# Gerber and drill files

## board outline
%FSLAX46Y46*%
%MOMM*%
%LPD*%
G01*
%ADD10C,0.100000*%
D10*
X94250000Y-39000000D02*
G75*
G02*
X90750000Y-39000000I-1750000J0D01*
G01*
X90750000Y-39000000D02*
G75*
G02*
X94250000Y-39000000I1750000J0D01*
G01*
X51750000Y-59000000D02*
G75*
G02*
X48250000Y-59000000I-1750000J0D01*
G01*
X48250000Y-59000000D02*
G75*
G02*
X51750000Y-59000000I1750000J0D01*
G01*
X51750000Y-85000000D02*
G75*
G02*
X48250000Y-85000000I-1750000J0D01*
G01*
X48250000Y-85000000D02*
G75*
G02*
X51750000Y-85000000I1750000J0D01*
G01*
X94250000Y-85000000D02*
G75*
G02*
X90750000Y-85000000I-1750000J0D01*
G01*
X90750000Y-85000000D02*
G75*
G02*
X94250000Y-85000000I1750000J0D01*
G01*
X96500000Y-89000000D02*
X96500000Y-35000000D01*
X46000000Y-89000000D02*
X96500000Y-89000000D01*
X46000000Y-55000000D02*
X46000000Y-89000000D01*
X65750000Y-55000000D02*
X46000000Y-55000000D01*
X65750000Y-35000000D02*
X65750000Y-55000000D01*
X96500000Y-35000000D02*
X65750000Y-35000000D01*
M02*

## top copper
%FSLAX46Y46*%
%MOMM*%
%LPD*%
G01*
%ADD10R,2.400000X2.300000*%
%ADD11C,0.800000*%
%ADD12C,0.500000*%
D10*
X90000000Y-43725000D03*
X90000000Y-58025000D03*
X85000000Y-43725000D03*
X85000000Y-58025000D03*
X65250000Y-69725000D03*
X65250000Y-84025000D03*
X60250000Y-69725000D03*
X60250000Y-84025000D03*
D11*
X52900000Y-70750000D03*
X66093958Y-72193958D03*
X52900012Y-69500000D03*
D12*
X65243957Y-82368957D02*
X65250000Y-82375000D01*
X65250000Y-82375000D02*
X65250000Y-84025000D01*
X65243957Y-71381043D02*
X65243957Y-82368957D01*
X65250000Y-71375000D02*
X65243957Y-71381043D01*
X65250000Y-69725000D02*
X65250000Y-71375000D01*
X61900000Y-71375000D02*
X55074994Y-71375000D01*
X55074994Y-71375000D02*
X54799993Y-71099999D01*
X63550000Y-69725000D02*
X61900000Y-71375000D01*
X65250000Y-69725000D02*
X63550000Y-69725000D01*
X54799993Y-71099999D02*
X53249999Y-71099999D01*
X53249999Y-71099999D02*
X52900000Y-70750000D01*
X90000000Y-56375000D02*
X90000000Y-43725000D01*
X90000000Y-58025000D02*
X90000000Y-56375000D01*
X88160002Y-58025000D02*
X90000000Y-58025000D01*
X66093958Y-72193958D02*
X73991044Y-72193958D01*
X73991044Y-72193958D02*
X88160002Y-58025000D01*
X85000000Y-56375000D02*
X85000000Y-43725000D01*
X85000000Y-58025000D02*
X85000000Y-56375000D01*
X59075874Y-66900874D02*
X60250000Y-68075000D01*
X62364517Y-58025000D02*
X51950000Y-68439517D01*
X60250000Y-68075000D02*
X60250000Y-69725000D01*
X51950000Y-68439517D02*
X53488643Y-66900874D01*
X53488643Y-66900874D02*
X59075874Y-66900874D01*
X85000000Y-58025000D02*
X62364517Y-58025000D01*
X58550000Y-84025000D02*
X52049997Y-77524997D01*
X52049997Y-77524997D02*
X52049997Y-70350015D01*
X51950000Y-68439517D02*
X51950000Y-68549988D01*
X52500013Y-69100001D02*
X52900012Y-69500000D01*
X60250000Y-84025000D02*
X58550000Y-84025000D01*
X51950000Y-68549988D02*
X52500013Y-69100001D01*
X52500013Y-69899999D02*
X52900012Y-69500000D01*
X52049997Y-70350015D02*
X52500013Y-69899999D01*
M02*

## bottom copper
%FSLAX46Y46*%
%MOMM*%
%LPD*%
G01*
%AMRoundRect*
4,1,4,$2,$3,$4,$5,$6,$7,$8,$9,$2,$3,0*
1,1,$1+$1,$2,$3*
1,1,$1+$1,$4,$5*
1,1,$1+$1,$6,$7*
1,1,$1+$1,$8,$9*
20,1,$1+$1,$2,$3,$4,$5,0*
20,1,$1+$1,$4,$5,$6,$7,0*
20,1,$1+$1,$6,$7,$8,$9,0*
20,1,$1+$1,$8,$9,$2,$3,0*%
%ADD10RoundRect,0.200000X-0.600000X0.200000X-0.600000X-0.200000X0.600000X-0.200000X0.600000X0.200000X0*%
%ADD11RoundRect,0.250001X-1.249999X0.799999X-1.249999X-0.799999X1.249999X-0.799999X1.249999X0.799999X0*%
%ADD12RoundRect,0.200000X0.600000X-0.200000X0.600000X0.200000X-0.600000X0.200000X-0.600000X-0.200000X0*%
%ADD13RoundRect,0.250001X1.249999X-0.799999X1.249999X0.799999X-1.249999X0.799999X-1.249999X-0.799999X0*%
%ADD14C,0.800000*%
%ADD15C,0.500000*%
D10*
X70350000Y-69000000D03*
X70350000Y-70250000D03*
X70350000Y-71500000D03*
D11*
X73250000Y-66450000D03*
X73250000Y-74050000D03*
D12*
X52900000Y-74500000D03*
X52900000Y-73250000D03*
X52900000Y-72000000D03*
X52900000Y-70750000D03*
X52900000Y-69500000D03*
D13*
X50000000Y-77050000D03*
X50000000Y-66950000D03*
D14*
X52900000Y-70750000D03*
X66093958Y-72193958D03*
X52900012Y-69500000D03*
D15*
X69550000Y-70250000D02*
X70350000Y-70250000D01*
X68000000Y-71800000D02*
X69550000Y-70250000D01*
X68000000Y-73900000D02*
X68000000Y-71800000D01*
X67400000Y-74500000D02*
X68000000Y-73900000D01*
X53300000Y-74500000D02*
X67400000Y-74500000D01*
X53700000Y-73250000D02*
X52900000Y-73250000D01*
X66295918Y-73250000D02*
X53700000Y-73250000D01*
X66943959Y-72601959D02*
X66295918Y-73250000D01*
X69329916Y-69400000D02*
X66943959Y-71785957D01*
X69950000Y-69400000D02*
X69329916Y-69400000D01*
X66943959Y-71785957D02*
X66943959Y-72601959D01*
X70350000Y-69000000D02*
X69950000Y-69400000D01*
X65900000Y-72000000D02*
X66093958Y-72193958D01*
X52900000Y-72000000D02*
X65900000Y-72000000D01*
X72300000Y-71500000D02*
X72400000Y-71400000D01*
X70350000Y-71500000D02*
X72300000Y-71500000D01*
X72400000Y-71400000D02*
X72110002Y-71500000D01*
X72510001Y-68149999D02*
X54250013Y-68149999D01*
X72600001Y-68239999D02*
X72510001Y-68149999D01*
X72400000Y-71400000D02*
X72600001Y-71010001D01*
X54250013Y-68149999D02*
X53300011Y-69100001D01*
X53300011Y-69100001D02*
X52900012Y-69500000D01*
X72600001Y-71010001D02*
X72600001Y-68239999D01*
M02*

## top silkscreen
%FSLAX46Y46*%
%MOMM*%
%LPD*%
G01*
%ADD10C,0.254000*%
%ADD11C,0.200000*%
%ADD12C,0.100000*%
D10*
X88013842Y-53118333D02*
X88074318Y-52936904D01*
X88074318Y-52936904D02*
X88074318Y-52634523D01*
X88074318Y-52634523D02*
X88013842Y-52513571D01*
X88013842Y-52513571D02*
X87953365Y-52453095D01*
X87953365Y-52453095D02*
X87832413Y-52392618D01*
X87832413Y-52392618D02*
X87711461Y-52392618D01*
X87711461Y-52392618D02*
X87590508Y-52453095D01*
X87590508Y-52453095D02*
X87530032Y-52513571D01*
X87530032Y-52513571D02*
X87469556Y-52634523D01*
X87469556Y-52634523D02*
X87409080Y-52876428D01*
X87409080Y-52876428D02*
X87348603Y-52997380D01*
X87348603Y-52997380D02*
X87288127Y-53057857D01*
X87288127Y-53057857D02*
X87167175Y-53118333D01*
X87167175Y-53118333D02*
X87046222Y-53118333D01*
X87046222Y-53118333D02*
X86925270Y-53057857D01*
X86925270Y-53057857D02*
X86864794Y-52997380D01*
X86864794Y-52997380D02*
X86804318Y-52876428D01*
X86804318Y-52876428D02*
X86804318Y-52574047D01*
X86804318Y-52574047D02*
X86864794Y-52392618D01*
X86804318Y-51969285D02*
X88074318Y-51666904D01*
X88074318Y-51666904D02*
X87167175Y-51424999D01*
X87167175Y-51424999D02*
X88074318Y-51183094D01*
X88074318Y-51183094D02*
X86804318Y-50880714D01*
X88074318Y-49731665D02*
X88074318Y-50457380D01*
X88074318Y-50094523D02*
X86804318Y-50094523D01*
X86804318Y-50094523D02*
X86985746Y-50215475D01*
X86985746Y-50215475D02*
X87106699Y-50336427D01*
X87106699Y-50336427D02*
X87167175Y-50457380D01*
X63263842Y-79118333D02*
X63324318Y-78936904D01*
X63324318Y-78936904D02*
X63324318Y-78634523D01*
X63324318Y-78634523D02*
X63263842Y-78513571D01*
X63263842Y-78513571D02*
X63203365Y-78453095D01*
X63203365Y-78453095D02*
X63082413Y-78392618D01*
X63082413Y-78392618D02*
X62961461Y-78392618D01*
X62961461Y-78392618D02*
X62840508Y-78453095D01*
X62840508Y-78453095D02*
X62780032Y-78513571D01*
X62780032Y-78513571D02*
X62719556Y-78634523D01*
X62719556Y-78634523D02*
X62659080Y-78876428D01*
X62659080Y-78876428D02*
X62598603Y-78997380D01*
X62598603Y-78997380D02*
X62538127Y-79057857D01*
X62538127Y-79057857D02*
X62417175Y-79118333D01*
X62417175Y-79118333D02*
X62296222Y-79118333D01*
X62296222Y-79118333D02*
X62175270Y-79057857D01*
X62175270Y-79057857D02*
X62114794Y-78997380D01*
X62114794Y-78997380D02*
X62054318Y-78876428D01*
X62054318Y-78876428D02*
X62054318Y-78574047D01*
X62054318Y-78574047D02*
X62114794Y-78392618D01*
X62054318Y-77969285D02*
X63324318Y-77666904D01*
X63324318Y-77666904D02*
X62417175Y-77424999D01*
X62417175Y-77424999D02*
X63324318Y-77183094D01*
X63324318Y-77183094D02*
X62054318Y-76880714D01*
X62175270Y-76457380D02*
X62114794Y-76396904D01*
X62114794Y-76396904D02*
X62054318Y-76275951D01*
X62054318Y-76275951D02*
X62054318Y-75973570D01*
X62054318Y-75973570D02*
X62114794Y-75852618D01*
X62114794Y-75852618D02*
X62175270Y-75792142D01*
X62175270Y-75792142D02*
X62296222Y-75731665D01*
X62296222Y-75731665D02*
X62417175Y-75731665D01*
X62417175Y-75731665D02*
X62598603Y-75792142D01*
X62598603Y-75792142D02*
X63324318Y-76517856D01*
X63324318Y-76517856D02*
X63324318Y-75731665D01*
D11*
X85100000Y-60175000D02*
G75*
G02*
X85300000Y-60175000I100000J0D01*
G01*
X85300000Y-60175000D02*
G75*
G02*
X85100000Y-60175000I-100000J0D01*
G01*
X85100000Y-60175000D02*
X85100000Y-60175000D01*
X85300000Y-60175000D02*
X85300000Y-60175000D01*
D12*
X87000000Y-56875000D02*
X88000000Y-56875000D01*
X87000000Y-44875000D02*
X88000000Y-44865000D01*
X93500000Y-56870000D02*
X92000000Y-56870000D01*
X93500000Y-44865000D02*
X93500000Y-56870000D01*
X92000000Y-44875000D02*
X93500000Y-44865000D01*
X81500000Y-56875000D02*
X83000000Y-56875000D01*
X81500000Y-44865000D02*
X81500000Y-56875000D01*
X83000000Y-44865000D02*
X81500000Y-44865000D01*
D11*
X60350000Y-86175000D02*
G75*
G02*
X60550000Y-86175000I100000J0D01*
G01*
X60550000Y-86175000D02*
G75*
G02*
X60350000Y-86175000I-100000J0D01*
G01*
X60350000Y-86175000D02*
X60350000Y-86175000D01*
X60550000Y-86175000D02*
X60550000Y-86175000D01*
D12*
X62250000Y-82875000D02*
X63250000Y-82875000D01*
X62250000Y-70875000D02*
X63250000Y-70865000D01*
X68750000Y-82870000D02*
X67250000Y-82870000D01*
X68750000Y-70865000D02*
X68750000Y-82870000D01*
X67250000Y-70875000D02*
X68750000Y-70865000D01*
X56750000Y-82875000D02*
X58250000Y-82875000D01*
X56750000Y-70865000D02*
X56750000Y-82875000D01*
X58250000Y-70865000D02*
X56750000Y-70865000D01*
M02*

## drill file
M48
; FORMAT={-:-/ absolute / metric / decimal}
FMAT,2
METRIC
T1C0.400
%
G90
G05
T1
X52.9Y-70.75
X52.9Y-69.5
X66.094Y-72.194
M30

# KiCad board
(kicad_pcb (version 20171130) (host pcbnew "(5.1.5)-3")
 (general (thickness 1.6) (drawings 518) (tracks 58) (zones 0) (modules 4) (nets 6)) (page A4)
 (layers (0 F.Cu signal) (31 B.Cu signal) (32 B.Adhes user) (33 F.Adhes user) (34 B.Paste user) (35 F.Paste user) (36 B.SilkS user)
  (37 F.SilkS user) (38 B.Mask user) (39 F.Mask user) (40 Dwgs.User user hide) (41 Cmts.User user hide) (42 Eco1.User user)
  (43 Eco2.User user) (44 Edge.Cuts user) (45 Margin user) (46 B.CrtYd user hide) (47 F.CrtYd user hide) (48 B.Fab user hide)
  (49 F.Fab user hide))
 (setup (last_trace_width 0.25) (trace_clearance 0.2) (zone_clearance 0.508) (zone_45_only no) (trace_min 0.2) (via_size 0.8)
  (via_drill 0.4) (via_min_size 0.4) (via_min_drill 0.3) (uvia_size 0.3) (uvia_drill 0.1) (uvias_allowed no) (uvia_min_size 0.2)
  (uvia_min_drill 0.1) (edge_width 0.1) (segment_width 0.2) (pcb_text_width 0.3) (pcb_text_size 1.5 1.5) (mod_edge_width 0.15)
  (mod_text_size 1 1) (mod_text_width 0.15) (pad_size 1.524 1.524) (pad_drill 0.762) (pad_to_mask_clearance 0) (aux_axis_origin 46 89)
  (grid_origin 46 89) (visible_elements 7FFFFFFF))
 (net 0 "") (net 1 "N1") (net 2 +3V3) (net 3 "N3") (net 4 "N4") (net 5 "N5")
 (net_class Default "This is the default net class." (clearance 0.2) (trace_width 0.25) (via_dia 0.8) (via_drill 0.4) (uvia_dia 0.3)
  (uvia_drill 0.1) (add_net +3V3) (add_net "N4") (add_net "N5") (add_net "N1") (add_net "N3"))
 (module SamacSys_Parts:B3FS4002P (layer F.Cu) (at 87.5 52 270)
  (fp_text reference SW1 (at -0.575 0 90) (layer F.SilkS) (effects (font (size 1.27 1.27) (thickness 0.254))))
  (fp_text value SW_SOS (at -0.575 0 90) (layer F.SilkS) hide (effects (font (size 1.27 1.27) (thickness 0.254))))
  (fp_arc (start 8.175 2.3) (end 8.175 2.4) (angle 180) (layer F.SilkS) (width 0.2))
  (fp_arc (start 8.175 2.3) (end 8.175 2.2) (angle 180) (layer F.SilkS) (width 0.2))
  (fp_line (start 8.175 2.4) (end 8.175 2.4) (layer F.SilkS) (width 0.2))
  (fp_line (start 8.175 2.2) (end 8.175 2.2) (layer F.SilkS) (width 0.2))
  (fp_line (start 4.875 0.5) (end 4.875 -0.5) (layer F.SilkS) (width 0.1))
  (fp_line (start -7.125 0.5) (end -7.135 -0.5) (layer F.SilkS) (width 0.1))
  (fp_line (start 4.87 -6) (end 4.87 -4.5) (layer F.SilkS) (width 0.1))
  (fp_line (start -7.135 -6) (end 4.87 -6) (layer F.SilkS) (width 0.1))
  (fp_line (start -7.125 -4.5) (end -7.135 -6) (layer F.SilkS) (width 0.1))
  (fp_line (start 4.875 6) (end 4.875 4.5) (layer F.SilkS) (width 0.1))
  (fp_line (start -7.135 6) (end 4.875 6) (layer F.SilkS) (width 0.1))
  (fp_line (start -7.135 4.5) (end -7.135 6) (layer F.SilkS) (width 0.1))
  (pad 2 smd rect (at -8.275 -2.5 270) (size 2.3 2.4) (layers F.Cu F.Paste F.Mask) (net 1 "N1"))
  (pad 2 smd rect (at 6.025 -2.5 270) (size 2.3 2.4) (layers F.Cu F.Paste F.Mask) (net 1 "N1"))
  (pad 1 smd rect (at -8.275 2.5 270) (size 2.3 2.4) (layers F.Cu F.Paste F.Mask) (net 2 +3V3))
  (pad 1 smd rect (at 6.025 2.5 270) (size 2.3 2.4) (layers F.Cu F.Paste F.Mask) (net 2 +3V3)))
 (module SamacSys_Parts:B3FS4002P (layer F.Cu) (at 62.75 78 270)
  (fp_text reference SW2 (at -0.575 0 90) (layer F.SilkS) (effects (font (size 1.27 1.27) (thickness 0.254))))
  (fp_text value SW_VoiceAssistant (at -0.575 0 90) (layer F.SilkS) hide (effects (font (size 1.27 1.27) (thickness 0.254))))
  (fp_arc (start 8.175 2.3) (end 8.175 2.4) (angle 180) (layer F.SilkS) (width 0.2))
  (fp_arc (start 8.175 2.3) (end 8.175 2.2) (angle 180) (layer F.SilkS) (width 0.2))
  (fp_line (start 8.175 2.4) (end 8.175 2.4) (layer F.SilkS) (width 0.2))
  (fp_line (start 8.175 2.2) (end 8.175 2.2) (layer F.SilkS) (width 0.2))
  (fp_line (start 4.875 0.5) (end 4.875 -0.5) (layer F.SilkS) (width 0.1))
  (fp_line (start -7.125 0.5) (end -7.135 -0.5) (layer F.SilkS) (width 0.1))
  (fp_line (start 4.87 -6) (end 4.87 -4.5) (layer F.SilkS) (width 0.1))
  (fp_line (start -7.135 -6) (end 4.87 -6) (layer F.SilkS) (width 0.1))
  (fp_line (start -7.125 -4.5) (end -7.135 -6) (layer F.SilkS) (width 0.1))
  (fp_line (start 4.875 6) (end 4.875 4.5) (layer F.SilkS) (width 0.1))
  (fp_line (start -7.135 6) (end 4.875 6) (layer F.SilkS) (width 0.1))
  (fp_line (start -7.135 4.5) (end -7.135 6) (layer F.SilkS) (width 0.1))
  (pad 2 smd rect (at -8.275 -2.5 270) (size 2.3 2.4) (layers F.Cu F.Paste F.Mask) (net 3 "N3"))
  (pad 2 smd rect (at 6.025 -2.5 270) (size 2.3 2.4) (layers F.Cu F.Paste F.Mask) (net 3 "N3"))
  (pad 1 smd rect (at -8.275 2.5 270) (size 2.3 2.4) (layers F.Cu F.Paste F.Mask) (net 2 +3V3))
  (pad 1 smd rect (at 6.025 2.5 270) (size 2.3 2.4) (layers F.Cu F.Paste F.Mask) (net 2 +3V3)))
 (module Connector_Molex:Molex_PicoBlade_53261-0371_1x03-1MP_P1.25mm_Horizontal (layer B.Cu) (at 72.75 70.25 270)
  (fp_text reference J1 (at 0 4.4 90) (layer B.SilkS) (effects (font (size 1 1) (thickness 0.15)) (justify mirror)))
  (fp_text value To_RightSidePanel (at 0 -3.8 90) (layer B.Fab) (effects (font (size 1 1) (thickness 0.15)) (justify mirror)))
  (pad 1 smd roundrect (at -1.25 2.4 270) (size 0.8 1.6) (layers B.Cu B.Paste B.Mask) (roundrect_rratio 0.25) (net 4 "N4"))
  (pad 2 smd roundrect (at 0 2.4 270) (size 0.8 1.6) (layers B.Cu B.Paste B.Mask) (roundrect_rratio 0.25) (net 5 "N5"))
  (pad 3 smd roundrect (at 1.25 2.4 270) (size 0.8 1.6) (layers B.Cu B.Paste B.Mask) (roundrect_rratio 0.25) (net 2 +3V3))
  (pad MP smd roundrect (at -3.8 -0.5 270) (size 2.1 3) (layers B.Cu B.Paste B.Mask) (roundrect_rratio 0.119048))
  (pad MP smd roundrect (at 3.8 -0.5 270) (size 2.1 3) (layers B.Cu B.Paste B.Mask) (roundrect_rratio 0.119048)))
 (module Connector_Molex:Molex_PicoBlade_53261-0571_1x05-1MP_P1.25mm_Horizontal (layer B.Cu) (at 50.5 72 90)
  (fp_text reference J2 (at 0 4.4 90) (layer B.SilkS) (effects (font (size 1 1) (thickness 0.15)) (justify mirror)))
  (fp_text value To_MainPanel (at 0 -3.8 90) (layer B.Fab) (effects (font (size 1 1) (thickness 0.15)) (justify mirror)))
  (pad 1 smd roundrect (at -2.5 2.4 90) (size 0.8 1.6) (layers B.Cu B.Paste B.Mask) (roundrect_rratio 0.25) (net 5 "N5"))
  (pad 2 smd roundrect (at -1.25 2.4 90) (size 0.8 1.6) (layers B.Cu B.Paste B.Mask) (roundrect_rratio 0.25) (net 4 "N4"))
  (pad 3 smd roundrect (at 0 2.4 90) (size 0.8 1.6) (layers B.Cu B.Paste B.Mask) (roundrect_rratio 0.25) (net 1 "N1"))
  (pad 4 smd roundrect (at 1.25 2.4 90) (size 0.8 1.6) (layers B.Cu B.Paste B.Mask) (roundrect_rratio 0.25) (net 3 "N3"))
  (pad 5 smd roundrect (at 2.5 2.4 90) (size 0.8 1.6) (layers B.Cu B.Paste B.Mask) (roundrect_rratio 0.25) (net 2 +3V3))
  (pad MP smd roundrect (at -5.05 -0.5 90) (size 2.1 3) (layers B.Cu B.Paste B.Mask) (roundrect_rratio 0.119048))
  (pad MP smd roundrect (at 5.05 -0.5 90) (size 2.1 3) (layers B.Cu B.Paste B.Mask) (roundrect_rratio 0.119048)))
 (gr_circle (center 92.5 39) (end 92.5 37.25) (layer Edge.Cuts) (width 0.1))
 (gr_circle (center 50 59) (end 48.25 59) (layer Edge.Cuts) (width 0.1))
 (gr_circle (center 50 85) (end 48.25 85) (layer Edge.Cuts) (width 0.1))
 (gr_circle (center 92.5 85) (end 90.75 85) (layer Edge.Cuts) (width 0.1))
 (gr_line (start 96.5 89) (end 96.5 35) (layer Edge.Cuts) (width 0.1))
 (gr_line (start 46 89) (end 96.5 89) (layer Edge.Cuts) (width 0.1))
 (gr_line (start 46 55) (end 46 89) (layer Edge.Cuts) (width 0.1))
 (gr_line (start 65.75 55) (end 46 55) (layer Edge.Cuts) (width 0.1))
 (gr_line (start 65.75 35) (end 65.75 55) (layer Edge.Cuts) (width 0.1))
 (gr_line (start 96.5 35) (end 65.75 35) (layer Edge.Cuts) (width 0.1))
 (segment (start 69.55 70.25) (end 70.35 70.25) (width 0.5) (layer B.Cu) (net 5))
 (segment (start 68 71.8) (end 69.55 70.25) (width 0.5) (layer B.Cu) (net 5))
 (segment (start 68 73.9) (end 68 71.8) (width 0.5) (layer B.Cu) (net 5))
 (segment (start 67.4 74.5) (end 68 73.9) (width 0.5) (layer B.Cu) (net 5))
 (segment (start 53.3 74.5) (end 67.4 74.5) (width 0.5) (layer B.Cu) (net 5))
 (segment (start 53.7 73.25) (end 52.9 73.25) (width 0.5) (layer B.Cu) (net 4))
 (segment (start 66.295918 73.25) (end 53.7 73.25) (width 0.5) (layer B.Cu) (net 4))
 (segment (start 66.943959 72.601959) (end 66.295918 73.25) (width 0.5) (layer B.Cu) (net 4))
 (segment (start 69.329916 69.4) (end 66.943959 71.785957) (width 0.5) (layer B.Cu) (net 4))
 (segment (start 69.95 69.4) (end 69.329916 69.4) (width 0.5) (layer B.Cu) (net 4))
 (segment (start 66.943959 71.785957) (end 66.943959 72.601959) (width 0.5) (layer B.Cu) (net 4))
 (segment (start 70.35 69) (end 69.95 69.4) (width 0.5) (layer B.Cu) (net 4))
 (segment (start 65.243957 82.368957) (end 65.25 82.375) (width 0.5) (layer F.Cu) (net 3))
 (segment (start 65.25 82.375) (end 65.25 84.025) (width 0.5) (layer F.Cu) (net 3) (status 20))
 (segment (start 65.243957 71.381043) (end 65.243957 82.368957) (width 0.5) (layer F.Cu) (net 3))
 (segment (start 65.25 71.375) (end 65.243957 71.381043) (width 0.5) (layer F.Cu) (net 3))
 (segment (start 65.25 69.725) (end 65.25 71.375) (width 0.5) (layer F.Cu) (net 3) (status 10))
 (segment (start 61.9 71.375) (end 55.074994 71.375) (width 0.5) (layer F.Cu) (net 3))
 (segment (start 55.074994 71.375) (end 54.799993 71.099999) (width 0.5) (layer F.Cu) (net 3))
 (segment (start 63.55 69.725) (end 61.9 71.375) (width 0.5) (layer F.Cu) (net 3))
 (segment (start 65.25 69.725) (end 63.55 69.725) (width 0.5) (layer F.Cu) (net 3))
 (via (at 52.9 70.75) (size 0.8) (drill 0.4) (layers F.Cu B.Cu) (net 3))
 (segment (start 54.799993 71.099999) (end 53.249999 71.099999) (width 0.5) (layer F.Cu) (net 3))
 (segment (start 53.249999 71.099999) (end 52.9 70.75) (width 0.5) (layer F.Cu) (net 3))
 (segment (start 90 56.375) (end 90 43.725) (width 0.5) (layer F.Cu) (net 1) (status 20))
 (segment (start 90 58.025) (end 90 56.375) (width 0.5) (layer F.Cu) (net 1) (status 10))
 (via (at 66.093958 72.193958) (size 0.8) (drill 0.4) (layers F.Cu B.Cu) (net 1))
 (segment (start 88.160002 58.025) (end 90 58.025) (width 0.5) (layer F.Cu) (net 1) (status 20))
 (segment (start 66.093958 72.193958) (end 73.991044 72.193958) (width 0.5) (layer F.Cu) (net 1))
 (segment (start 73.991044 72.193958) (end 88.160002 58.025) (width 0.5) (layer F.Cu) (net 1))
 (segment (start 65.9 72) (end 66.093958 72.193958) (width 0.5) (layer B.Cu) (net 1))
 (segment (start 52.9 72) (end 65.9 72) (width 0.5) (layer B.Cu) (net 1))
 (segment (start 85 56.375) (end 85 43.725) (width 0.5) (layer F.Cu) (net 2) (status 20))
 (segment (start 85 58.025) (end 85 56.375) (width 0.5) (layer F.Cu) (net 2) (status 10))
 (segment (start 59.075874 66.900874) (end 60.25 68.075) (width 0.5) (layer F.Cu) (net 2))
 (segment (start 62.364517 58.025) (end 51.95 68.439517) (width 0.5) (layer F.Cu) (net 2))
 (segment (start 60.25 68.075) (end 60.25 69.725) (width 0.5) (layer F.Cu) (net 2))
 (segment (start 51.95 68.439517) (end 53.488643 66.900874) (width 0.5) (layer F.Cu) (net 2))
 (segment (start 53.488643 66.900874) (end 59.075874 66.900874) (width 0.5) (layer F.Cu) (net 2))
 (segment (start 85 58.025) (end 62.364517 58.025) (width 0.5) (layer F.Cu) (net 2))
 (segment (start 72.3 71.5) (end 72.4 71.4) (width 0.5) (layer B.Cu) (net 2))
 (segment (start 70.35 71.5) (end 72.3 71.5) (width 0.5) (layer B.Cu) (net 2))
 (segment (start 72.4 71.4) (end 72.110002 71.5) (width 0.5) (layer B.Cu) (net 2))
 (via (at 52.900012 69.5) (size 0.8) (drill 0.4) (layers F.Cu B.Cu) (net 2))
 (segment (start 58.55 84.025) (end 52.049997 77.524997) (width 0.5) (layer F.Cu) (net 2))
 (segment (start 52.049997 77.524997) (end 52.049997 70.350015) (width 0.5) (layer F.Cu) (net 2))
 (segment (start 72.510001 68.149999) (end 54.250013 68.149999) (width 0.5) (layer B.Cu) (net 2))
 (segment (start 72.600001 68.239999) (end 72.510001 68.149999) (width 0.5) (layer B.Cu) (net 2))
 (segment (start 51.95 68.439517) (end 51.95 68.549988) (width 0.5) (layer F.Cu) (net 2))
 (segment (start 72.4 71.4) (end 72.600001 71.010001) (width 0.5) (layer B.Cu) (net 2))
 (segment (start 52.500013 69.100001) (end 52.900012 69.5) (width 0.5) (layer F.Cu) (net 2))
 (segment (start 54.250013 68.149999) (end 53.300011 69.100001) (width 0.5) (layer B.Cu) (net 2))
 (segment (start 60.25 84.025) (end 58.55 84.025) (width 0.5) (layer F.Cu) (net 2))
 (segment (start 51.95 68.549988) (end 52.500013 69.100001) (width 0.5) (layer F.Cu) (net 2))
 (segment (start 53.300011 69.100001) (end 52.900012 69.5) (width 0.5) (layer B.Cu) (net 2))
 (segment (start 52.500013 69.899999) (end 52.900012 69.5) (width 0.5) (layer F.Cu) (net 2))
 (segment (start 52.049997 70.350015) (end 52.500013 69.899999) (width 0.5) (layer F.Cu) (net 2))
 (segment (start 72.600001 71.010001) (end 72.600001 68.239999) (width 0.5) (layer B.Cu) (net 2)))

